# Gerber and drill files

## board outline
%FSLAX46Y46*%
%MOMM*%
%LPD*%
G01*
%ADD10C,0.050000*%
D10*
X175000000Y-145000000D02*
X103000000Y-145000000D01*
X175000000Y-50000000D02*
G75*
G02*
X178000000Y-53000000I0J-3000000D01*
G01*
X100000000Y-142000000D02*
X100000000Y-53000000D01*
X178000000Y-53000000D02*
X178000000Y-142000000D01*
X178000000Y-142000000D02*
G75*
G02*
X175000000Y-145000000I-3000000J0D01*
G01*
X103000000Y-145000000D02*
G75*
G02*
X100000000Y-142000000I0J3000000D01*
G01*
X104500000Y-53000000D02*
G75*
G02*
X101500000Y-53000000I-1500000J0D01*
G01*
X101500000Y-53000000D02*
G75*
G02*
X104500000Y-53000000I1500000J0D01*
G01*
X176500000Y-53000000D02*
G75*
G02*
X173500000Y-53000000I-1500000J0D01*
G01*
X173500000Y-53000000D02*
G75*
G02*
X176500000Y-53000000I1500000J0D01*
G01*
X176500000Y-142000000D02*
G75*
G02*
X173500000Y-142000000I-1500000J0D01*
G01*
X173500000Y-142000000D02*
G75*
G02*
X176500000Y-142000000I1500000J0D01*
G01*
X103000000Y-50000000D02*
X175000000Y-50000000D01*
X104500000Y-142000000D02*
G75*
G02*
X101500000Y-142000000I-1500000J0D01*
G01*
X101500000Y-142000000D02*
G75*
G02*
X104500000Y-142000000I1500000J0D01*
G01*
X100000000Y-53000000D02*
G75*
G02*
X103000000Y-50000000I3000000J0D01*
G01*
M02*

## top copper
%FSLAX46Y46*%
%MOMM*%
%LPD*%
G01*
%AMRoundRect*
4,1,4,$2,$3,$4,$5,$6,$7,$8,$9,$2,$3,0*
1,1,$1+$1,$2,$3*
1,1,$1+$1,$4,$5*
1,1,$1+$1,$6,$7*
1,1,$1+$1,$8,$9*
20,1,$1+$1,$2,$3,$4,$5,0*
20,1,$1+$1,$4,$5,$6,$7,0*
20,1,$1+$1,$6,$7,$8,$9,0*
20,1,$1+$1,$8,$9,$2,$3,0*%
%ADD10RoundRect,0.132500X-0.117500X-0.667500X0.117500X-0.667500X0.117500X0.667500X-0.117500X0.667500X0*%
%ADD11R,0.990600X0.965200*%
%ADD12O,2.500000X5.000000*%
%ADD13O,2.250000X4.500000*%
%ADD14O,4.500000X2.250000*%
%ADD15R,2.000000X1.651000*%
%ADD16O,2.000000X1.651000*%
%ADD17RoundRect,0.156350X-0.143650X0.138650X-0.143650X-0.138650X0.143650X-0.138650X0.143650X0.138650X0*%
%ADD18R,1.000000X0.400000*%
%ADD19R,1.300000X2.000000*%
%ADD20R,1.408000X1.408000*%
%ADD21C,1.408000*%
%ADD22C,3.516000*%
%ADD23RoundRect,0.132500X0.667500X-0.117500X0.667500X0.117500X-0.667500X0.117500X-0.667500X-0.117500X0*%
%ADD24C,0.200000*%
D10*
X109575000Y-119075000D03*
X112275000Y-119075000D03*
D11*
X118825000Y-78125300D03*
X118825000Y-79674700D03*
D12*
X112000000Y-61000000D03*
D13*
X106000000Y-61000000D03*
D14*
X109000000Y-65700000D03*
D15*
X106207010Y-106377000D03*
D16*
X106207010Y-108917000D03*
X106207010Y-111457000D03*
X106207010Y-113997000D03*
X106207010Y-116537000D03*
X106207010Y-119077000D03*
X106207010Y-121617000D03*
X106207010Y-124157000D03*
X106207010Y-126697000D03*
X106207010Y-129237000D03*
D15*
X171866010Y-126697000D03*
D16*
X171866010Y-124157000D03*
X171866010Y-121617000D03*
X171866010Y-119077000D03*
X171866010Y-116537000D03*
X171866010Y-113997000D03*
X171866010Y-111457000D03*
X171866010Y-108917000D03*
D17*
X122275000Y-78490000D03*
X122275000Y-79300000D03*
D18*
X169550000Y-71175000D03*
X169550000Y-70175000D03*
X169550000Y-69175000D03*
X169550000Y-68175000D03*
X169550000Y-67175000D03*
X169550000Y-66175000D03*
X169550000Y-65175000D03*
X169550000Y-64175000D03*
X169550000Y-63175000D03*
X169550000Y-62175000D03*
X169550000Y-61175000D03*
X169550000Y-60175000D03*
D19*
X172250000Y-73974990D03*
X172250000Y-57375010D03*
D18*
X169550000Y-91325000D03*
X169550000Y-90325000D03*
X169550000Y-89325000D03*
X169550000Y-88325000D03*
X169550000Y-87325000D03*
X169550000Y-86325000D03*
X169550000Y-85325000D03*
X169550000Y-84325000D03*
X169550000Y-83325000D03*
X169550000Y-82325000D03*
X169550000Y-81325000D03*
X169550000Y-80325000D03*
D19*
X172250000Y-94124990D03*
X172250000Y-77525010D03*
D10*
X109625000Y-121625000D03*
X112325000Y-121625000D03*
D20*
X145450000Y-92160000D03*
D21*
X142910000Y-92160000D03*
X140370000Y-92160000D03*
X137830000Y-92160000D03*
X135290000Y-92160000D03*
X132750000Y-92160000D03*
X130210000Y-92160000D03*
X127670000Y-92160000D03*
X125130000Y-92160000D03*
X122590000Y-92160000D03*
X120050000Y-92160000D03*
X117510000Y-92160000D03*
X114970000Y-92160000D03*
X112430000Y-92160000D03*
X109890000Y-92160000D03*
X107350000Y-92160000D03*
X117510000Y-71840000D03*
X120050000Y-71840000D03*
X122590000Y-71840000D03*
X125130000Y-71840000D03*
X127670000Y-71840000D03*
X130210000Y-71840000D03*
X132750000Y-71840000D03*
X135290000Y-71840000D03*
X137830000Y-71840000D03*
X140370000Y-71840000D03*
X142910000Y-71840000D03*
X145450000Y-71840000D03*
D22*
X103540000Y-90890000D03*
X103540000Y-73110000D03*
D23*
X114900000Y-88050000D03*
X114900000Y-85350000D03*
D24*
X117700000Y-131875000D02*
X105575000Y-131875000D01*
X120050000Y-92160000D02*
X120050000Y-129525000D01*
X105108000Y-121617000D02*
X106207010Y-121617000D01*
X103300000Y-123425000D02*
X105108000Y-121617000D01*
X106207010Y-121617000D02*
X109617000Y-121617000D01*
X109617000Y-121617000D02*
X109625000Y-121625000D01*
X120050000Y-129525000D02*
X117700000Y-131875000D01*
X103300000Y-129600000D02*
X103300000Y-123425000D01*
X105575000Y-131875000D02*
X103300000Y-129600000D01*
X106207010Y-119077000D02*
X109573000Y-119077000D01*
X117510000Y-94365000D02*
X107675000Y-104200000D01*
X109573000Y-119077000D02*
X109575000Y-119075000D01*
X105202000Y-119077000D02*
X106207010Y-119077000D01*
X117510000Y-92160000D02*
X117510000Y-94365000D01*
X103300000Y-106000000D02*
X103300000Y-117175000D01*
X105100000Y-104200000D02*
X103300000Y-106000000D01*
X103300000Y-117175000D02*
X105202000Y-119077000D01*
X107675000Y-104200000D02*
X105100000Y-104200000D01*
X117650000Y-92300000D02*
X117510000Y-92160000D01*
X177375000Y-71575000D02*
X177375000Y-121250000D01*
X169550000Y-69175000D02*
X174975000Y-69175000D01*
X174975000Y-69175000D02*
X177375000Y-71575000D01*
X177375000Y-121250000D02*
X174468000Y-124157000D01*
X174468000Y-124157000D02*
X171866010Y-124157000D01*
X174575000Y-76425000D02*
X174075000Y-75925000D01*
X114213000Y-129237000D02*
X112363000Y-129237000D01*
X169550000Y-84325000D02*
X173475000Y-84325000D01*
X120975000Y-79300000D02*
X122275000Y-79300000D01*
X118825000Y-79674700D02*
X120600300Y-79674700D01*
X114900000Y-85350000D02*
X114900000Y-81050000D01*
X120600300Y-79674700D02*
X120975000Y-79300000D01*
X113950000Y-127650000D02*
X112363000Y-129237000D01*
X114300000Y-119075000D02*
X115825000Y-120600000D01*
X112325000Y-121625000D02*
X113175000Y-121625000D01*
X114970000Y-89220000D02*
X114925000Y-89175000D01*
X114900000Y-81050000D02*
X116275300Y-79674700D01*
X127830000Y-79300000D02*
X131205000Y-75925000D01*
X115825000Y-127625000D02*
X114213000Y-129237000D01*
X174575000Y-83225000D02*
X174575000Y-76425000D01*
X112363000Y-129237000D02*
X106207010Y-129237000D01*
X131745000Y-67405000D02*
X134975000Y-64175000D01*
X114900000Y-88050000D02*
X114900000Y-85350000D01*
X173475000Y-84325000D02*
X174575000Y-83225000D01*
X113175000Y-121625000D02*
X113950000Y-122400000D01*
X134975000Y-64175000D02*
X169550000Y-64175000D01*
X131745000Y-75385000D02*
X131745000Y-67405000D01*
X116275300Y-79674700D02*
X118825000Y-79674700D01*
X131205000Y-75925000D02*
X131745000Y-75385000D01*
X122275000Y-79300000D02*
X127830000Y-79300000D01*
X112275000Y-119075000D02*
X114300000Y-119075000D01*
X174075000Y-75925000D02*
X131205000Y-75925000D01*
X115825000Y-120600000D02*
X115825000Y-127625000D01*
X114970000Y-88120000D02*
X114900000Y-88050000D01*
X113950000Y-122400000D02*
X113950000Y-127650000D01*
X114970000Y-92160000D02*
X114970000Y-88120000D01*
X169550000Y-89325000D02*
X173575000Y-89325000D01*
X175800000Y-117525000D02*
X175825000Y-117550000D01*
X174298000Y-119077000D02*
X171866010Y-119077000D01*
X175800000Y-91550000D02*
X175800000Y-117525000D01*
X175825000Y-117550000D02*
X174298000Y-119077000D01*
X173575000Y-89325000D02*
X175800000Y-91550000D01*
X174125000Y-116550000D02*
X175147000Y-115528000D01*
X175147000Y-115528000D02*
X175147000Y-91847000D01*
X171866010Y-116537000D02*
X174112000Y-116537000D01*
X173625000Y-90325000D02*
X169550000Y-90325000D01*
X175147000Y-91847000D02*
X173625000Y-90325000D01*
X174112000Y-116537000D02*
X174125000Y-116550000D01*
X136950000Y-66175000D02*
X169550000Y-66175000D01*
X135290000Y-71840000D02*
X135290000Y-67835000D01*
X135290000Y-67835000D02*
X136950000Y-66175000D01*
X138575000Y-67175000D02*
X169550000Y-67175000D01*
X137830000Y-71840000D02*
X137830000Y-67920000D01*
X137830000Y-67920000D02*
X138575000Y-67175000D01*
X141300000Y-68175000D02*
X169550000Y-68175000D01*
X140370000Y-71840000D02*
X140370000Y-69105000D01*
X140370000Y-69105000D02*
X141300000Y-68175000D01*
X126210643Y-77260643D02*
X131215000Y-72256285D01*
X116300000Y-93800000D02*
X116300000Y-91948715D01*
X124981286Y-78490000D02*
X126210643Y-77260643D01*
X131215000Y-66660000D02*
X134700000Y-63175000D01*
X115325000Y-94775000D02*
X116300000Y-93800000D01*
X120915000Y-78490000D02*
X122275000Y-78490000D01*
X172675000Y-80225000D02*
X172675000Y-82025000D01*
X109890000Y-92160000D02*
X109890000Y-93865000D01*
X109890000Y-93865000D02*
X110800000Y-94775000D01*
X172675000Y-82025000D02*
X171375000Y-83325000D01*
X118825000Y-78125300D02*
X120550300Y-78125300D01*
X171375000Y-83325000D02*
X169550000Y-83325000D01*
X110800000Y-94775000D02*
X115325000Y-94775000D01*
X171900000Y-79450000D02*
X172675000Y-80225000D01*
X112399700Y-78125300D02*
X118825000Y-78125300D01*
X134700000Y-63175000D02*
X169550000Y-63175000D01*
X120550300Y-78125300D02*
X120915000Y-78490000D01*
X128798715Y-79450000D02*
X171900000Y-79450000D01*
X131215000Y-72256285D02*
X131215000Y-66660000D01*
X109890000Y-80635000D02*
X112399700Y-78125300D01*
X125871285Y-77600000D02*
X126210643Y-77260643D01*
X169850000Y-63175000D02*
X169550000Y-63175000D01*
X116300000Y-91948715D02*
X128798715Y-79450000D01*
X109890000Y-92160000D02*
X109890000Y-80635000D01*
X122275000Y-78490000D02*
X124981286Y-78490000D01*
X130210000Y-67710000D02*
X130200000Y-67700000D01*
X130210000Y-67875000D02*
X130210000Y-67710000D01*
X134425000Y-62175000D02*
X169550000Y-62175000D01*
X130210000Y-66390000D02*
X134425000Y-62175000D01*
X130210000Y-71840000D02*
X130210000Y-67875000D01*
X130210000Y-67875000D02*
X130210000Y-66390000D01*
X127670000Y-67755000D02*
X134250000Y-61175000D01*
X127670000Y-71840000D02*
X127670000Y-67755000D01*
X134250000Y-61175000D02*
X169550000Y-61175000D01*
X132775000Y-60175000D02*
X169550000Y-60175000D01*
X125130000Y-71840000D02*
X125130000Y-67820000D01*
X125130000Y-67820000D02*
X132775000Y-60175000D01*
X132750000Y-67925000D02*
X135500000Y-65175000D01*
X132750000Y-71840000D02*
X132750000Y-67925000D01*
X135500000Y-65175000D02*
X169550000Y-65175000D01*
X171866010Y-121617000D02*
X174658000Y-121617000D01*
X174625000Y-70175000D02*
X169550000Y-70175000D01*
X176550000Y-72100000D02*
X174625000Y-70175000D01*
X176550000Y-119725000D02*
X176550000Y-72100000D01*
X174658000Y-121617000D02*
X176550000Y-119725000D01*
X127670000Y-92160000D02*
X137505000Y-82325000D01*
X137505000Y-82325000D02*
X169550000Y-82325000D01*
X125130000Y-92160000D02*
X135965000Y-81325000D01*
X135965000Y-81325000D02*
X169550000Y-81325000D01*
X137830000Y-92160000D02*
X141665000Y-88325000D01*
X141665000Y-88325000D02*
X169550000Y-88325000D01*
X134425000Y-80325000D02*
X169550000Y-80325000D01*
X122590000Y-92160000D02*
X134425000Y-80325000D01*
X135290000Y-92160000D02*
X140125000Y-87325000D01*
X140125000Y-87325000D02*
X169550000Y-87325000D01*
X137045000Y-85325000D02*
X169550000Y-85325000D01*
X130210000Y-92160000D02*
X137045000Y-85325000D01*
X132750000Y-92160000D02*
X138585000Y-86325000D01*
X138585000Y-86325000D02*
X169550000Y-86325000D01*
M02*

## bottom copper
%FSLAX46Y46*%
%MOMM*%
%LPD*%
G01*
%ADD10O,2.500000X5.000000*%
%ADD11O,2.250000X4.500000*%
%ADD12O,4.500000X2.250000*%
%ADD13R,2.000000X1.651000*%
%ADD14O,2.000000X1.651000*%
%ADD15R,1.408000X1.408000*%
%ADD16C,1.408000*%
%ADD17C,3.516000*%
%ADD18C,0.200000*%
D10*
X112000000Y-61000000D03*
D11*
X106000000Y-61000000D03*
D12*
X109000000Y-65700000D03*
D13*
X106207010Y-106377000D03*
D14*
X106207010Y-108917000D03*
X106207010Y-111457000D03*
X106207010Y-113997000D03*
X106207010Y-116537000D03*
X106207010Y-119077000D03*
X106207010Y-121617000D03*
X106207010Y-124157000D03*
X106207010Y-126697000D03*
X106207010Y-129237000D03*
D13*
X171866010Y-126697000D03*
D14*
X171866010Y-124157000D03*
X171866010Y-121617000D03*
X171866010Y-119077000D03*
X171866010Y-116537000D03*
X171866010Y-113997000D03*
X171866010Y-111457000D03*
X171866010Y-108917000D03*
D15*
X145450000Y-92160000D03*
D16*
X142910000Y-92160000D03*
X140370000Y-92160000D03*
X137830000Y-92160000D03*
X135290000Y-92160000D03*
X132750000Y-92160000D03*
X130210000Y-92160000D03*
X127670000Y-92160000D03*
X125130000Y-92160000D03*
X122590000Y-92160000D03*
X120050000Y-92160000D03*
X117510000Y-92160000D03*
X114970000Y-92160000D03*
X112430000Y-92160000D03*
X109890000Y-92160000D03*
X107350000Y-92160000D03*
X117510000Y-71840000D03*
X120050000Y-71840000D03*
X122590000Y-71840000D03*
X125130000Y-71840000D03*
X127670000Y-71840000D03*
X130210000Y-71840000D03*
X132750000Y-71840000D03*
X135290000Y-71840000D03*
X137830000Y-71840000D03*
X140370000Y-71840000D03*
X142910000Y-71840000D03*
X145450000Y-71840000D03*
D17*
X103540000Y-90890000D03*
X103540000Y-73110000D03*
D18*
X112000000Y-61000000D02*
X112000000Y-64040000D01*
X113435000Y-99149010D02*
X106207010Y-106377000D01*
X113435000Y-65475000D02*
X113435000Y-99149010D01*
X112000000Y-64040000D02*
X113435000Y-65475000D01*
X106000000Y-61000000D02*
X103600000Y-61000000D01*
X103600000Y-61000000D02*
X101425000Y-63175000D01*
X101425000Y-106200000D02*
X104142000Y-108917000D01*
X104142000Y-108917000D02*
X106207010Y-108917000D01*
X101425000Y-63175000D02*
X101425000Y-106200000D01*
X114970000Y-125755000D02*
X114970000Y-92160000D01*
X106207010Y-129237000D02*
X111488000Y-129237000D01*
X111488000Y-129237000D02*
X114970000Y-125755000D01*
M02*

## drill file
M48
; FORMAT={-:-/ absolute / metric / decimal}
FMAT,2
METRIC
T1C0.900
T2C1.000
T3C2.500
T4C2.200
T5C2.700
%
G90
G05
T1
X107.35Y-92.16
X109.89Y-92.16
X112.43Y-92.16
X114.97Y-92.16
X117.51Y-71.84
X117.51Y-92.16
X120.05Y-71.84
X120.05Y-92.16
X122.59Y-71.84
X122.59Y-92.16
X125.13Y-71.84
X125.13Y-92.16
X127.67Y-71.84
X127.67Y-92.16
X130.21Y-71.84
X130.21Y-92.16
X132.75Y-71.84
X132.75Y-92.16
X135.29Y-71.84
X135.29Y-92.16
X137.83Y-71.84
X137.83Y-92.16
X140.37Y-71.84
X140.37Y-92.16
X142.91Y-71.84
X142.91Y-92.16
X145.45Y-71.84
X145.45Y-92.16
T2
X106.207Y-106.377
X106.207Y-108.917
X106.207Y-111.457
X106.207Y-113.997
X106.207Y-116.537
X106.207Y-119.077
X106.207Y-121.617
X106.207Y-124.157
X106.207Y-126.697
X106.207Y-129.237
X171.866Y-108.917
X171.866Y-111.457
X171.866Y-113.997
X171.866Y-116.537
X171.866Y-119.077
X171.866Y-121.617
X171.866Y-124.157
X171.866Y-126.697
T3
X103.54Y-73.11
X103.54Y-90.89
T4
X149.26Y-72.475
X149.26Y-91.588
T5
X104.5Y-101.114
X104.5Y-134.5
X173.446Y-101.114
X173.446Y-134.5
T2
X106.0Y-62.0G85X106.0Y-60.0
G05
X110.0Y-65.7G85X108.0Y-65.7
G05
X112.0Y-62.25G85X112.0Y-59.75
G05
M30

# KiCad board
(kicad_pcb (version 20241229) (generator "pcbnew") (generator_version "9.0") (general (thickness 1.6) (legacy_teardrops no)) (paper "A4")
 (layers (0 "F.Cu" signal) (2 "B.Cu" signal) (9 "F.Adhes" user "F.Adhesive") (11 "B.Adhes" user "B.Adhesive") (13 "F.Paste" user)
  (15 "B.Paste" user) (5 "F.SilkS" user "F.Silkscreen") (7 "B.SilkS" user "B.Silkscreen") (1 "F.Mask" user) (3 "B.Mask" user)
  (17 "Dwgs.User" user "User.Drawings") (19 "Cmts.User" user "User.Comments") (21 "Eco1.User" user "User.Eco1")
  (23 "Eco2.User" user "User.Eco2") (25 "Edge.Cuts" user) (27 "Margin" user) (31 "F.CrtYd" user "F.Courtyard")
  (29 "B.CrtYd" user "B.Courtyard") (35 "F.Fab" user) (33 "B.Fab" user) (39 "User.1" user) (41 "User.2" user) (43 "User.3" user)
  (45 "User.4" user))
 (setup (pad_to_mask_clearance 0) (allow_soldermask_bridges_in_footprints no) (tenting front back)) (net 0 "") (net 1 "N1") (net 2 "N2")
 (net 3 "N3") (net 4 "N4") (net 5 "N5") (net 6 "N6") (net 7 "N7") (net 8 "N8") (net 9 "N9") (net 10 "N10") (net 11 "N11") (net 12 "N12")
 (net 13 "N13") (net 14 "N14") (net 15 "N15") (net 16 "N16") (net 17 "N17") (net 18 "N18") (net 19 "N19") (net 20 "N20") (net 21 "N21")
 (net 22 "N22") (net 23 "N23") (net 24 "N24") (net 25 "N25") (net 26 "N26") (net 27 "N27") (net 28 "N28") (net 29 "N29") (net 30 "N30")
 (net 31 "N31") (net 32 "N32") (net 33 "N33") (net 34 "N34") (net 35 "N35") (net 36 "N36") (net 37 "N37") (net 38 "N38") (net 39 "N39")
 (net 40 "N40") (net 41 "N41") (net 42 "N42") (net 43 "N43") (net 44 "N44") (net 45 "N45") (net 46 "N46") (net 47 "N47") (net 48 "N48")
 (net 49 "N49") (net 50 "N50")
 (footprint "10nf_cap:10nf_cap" (layer "F.Cu") (at 109.575 119.075)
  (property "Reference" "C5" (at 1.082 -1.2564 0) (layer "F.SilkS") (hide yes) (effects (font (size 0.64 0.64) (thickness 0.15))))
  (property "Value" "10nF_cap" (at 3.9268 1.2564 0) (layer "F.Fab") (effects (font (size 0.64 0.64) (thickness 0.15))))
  (pad "1" smd roundrect (at 0 0) (size 0.5 1.6) (layers "F.Cu" "F.Mask" "F.Paste") (roundrect_rratio 0.265) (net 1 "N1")
   (solder_mask_margin 0.102))
  (pad "2" smd roundrect (at 2.7 0) (size 0.5 1.6) (layers "F.Cu" "F.Mask" "F.Paste") (roundrect_rratio 0.265) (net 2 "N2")
   (solder_mask_margin 0.102)))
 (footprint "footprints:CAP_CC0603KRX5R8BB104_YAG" (layer "F.Cu") (at 118.825 78.9 -90)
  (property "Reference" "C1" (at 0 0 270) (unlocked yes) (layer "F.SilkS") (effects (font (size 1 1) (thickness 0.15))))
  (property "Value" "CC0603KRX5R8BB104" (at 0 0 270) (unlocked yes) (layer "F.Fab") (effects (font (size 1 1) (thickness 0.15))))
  (pad "1" smd rect (at -0.7747 0 270) (size 0.9652 0.9906) (layers "F.Cu" "F.Mask" "F.Paste") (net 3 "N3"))
  (pad "2" smd rect (at 0.7747 0 270) (size 0.9652 0.9906) (layers "F.Cu" "F.Mask" "F.Paste") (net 2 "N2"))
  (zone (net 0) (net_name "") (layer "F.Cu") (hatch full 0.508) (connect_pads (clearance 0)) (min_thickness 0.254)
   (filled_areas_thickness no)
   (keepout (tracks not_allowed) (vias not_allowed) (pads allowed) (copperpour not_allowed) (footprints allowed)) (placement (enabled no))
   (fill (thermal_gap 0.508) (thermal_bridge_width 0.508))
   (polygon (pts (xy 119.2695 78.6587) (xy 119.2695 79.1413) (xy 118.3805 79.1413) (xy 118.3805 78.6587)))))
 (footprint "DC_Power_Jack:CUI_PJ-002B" (layer "F.Cu") (at 112 61 180)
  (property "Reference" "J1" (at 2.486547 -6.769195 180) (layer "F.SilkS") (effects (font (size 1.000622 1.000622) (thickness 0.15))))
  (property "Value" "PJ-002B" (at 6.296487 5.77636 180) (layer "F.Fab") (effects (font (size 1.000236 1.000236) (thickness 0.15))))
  (pad "1" thru_hole oval (at 0 0 180) (size 2.5 5) (drill oval 1 3.5) (layers "*.Cu" "*.Mask") (remove_unused_layers no) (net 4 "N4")
   (solder_mask_margin 0.102))
  (pad "2" thru_hole oval (at 6 0 180) (size 2.25 4.5) (drill oval 1 3) (layers "*.Cu" "*.Mask") (remove_unused_layers no) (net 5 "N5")
   (solder_mask_margin 0.102))
  (pad "3" thru_hole oval (at 3 -4.7 180) (size 4.5 2.25) (drill oval 3 1) (layers "*.Cu" "*.Mask") (remove_unused_layers no) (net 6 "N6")
   (solder_mask_margin 0.102)))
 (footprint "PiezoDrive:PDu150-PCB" (layer "F.Cu") (at 101 138)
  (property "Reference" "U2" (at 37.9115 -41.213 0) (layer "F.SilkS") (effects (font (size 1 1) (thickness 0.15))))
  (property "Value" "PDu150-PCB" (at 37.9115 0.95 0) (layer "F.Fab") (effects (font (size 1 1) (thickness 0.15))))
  (pad "" np_thru_hole circle (at 3.5 -36.886 270) (size 1.524 1.524) (drill 2.7) (layers "*.Cu" "*.Mask") (thermal_bridge_angle 90))
  (pad "" np_thru_hole circle (at 3.5 -3.5) (size 1.524 1.524) (drill 2.7) (layers "*.Cu" "*.Mask") (thermal_bridge_angle 90))
  (pad "" np_thru_hole circle (at 72.446 -36.886 180) (size 1.524 1.524) (drill 2.7) (layers "*.Cu" "*.Mask") (thermal_bridge_angle 90))
  (pad "" np_thru_hole circle (at 72.446 -3.5 90) (size 1.524 1.524) (drill 2.7) (layers "*.Cu" "*.Mask") (thermal_bridge_angle 90))
  (pad "1" thru_hole rect (at 5.20701 -31.623 270) (size 1.651 2) (drill 1) (layers "*.Cu" "*.Mask") (remove_unused_layers no) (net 4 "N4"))
  (pad "2" thru_hole oval (at 5.20701 -29.083 270) (size 1.651 2) (drill 1) (layers "*.Cu" "*.Mask") (remove_unused_layers no) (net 5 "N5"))
  (pad "3" thru_hole oval (at 5.20701 -26.543 270) (size 1.651 2) (drill 1) (layers "*.Cu" "*.Mask") (remove_unused_layers no) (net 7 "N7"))
  (pad "4" thru_hole oval (at 5.20701 -24.003 270) (size 1.651 2) (drill 1) (layers "*.Cu" "*.Mask") (remove_unused_layers no) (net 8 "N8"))
  (pad "5" thru_hole oval (at 5.20701 -21.463 270) (size 1.651 2) (drill 1) (layers "*.Cu" "*.Mask") (remove_unused_layers no) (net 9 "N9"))
  (pad "6" thru_hole oval (at 5.20701 -18.923 270) (size 1.651 2) (drill 1) (layers "*.Cu" "*.Mask") (remove_unused_layers no) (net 1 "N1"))
  (pad "7" thru_hole oval (at 5.20701 -16.383 270) (size 1.651 2) (drill 1) (layers "*.Cu" "*.Mask") (remove_unused_layers no)
   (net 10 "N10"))
  (pad "8" thru_hole oval (at 5.20701 -13.843 270) (size 1.651 2) (drill 1) (layers "*.Cu" "*.Mask") (remove_unused_layers no)
   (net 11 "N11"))
  (pad "9" thru_hole oval (at 5.20701 -11.303 270) (size 1.651 2) (drill 1) (layers "*.Cu" "*.Mask") (remove_unused_layers no)
   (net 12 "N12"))
  (pad "10" thru_hole oval (at 5.20701 -8.763 270) (size 1.651 2) (drill 1) (layers "*.Cu" "*.Mask") (remove_unused_layers no) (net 2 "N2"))
  (pad "11" thru_hole rect (at 70.86601 -11.303 90) (size 1.651 2) (drill 1) (layers "*.Cu" "*.Mask") (remove_unused_layers no)
   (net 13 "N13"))
  (pad "12" thru_hole oval (at 70.86601 -13.843 90) (size 1.651 2) (drill 1) (layers "*.Cu" "*.Mask") (remove_unused_layers no)
   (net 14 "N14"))
  (pad "13" thru_hole oval (at 70.86601 -16.383 90) (size 1.651 2) (drill 1) (layers "*.Cu" "*.Mask") (remove_unused_layers no)
   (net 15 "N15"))
  (pad "14" thru_hole oval (at 70.86601 -18.923 90) (size 1.651 2) (drill 1) (layers "*.Cu" "*.Mask") (remove_unused_layers no)
   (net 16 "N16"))
  (pad "15" thru_hole oval (at 70.86601 -21.463 90) (size 1.651 2) (drill 1) (layers "*.Cu" "*.Mask") (remove_unused_layers no)
   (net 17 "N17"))
  (pad "16" thru_hole oval (at 70.86601 -24.003 90) (size 1.651 2) (drill 1) (layers "*.Cu" "*.Mask") (remove_unused_layers no)
   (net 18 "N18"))
  (pad "17" thru_hole oval (at 70.86601 -26.543 90) (size 1.651 2) (drill 1) (layers "*.Cu" "*.Mask") (remove_unused_layers no)
   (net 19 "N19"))
  (pad "18" thru_hole oval (at 70.86601 -29.083 90) (size 1.651 2) (drill 1) (layers "*.Cu" "*.Mask") (remove_unused_layers no)
   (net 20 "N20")))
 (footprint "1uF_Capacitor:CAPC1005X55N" (layer "F.Cu") (at 122.275 78.895 -90)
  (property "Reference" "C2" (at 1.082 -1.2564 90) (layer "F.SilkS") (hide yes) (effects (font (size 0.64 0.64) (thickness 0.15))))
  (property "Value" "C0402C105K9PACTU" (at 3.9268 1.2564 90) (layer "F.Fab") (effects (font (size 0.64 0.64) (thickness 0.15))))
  (pad "1" smd roundrect (at -0.405 0 270) (size 0.59 0.6) (layers "F.Cu" "F.Mask" "F.Paste") (roundrect_rratio 0.265) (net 3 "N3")
   (solder_mask_margin 0.102))
  (pad "2" smd roundrect (at 0.405 0 270) (size 0.59 0.6) (layers "F.Cu" "F.Mask" "F.Paste") (roundrect_rratio 0.265) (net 2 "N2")
   (solder_mask_margin 0.102)))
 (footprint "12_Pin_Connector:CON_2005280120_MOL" (layer "F.Cu") (at 172 65.675 90)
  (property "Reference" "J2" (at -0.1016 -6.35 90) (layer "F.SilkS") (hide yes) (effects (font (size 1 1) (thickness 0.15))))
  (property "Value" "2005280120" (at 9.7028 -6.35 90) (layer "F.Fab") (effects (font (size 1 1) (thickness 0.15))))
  (pad "1" smd rect (at -5.5 -2.45 90) (size 0.4 1) (layers "F.Cu" "F.Mask" "F.Paste") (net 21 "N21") (solder_mask_margin 0.102))
  (pad "2" smd rect (at -4.5 -2.45 90) (size 0.4 1) (layers "F.Cu" "F.Mask" "F.Paste") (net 15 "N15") (solder_mask_margin 0.102))
  (pad "3" smd rect (at -3.5 -2.45 90) (size 0.4 1) (layers "F.Cu" "F.Mask" "F.Paste") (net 14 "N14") (solder_mask_margin 0.102))
  (pad "4" smd rect (at -2.5 -2.45 90) (size 0.4 1) (layers "F.Cu" "F.Mask" "F.Paste") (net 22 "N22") (solder_mask_margin 0.102))
  (pad "5" smd rect (at -1.5 -2.45 90) (size 0.4 1) (layers "F.Cu" "F.Mask" "F.Paste") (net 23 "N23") (solder_mask_margin 0.102))
  (pad "6" smd rect (at -0.5 -2.45 90) (size 0.4 1) (layers "F.Cu" "F.Mask" "F.Paste") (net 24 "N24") (solder_mask_margin 0.102))
  (pad "7" smd rect (at 0.5 -2.45 90) (size 0.4 1) (layers "F.Cu" "F.Mask" "F.Paste") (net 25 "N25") (solder_mask_margin 0.102))
  (pad "8" smd rect (at 1.5 -2.45 90) (size 0.4 1) (layers "F.Cu" "F.Mask" "F.Paste") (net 2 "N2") (solder_mask_margin 0.102))
  (pad "9" smd rect (at 2.5 -2.45 90) (size 0.4 1) (layers "F.Cu" "F.Mask" "F.Paste") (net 3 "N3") (solder_mask_margin 0.102))
  (pad "10" smd rect (at 3.5 -2.45 90) (size 0.4 1) (layers "F.Cu" "F.Mask" "F.Paste") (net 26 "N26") (solder_mask_margin 0.102))
  (pad "11" smd rect (at 4.5 -2.45 90) (size 0.4 1) (layers "F.Cu" "F.Mask" "F.Paste") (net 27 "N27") (solder_mask_margin 0.102))
  (pad "12" smd rect (at 5.5 -2.45 90) (size 0.4 1) (layers "F.Cu" "F.Mask" "F.Paste") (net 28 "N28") (solder_mask_margin 0.102))
  (pad "P1" smd rect (at -8.29999 0.25 90) (size 2 1.3) (layers "F.Cu" "F.Mask" "F.Paste") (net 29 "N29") (solder_mask_margin 0.102))
  (pad "P2" smd rect (at 8.29999 0.25 90) (size 2 1.3) (layers "F.Cu" "F.Mask" "F.Paste") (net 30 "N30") (solder_mask_margin 0.102)))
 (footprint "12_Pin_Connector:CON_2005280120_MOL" (layer "F.Cu") (at 172 85.825 90)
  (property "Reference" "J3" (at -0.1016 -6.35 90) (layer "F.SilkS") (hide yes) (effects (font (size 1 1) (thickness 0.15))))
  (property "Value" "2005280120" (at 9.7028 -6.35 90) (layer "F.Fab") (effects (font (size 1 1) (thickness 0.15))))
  (pad "1" smd rect (at -5.5 -2.45 90) (size 0.4 1) (layers "F.Cu" "F.Mask" "F.Paste") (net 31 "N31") (solder_mask_margin 0.102))
  (pad "2" smd rect (at -4.5 -2.45 90) (size 0.4 1) (layers "F.Cu" "F.Mask" "F.Paste") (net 17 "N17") (solder_mask_margin 0.102))
  (pad "3" smd rect (at -3.5 -2.45 90) (size 0.4 1) (layers "F.Cu" "F.Mask" "F.Paste") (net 16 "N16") (solder_mask_margin 0.102))
  (pad "4" smd rect (at -2.5 -2.45 90) (size 0.4 1) (layers "F.Cu" "F.Mask" "F.Paste") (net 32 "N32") (solder_mask_margin 0.102))
  (pad "5" smd rect (at -1.5 -2.45 90) (size 0.4 1) (layers "F.Cu" "F.Mask" "F.Paste") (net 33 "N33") (solder_mask_margin 0.102))
  (pad "6" smd rect (at -0.5 -2.45 90) (size 0.4 1) (layers "F.Cu" "F.Mask" "F.Paste") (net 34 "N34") (solder_mask_margin 0.102))
  (pad "7" smd rect (at 0.5 -2.45 90) (size 0.4 1) (layers "F.Cu" "F.Mask" "F.Paste") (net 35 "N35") (solder_mask_margin 0.102))
  (pad "8" smd rect (at 1.5 -2.45 90) (size 0.4 1) (layers "F.Cu" "F.Mask" "F.Paste") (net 2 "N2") (solder_mask_margin 0.102))
  (pad "9" smd rect (at 2.5 -2.45 90) (size 0.4 1) (layers "F.Cu" "F.Mask" "F.Paste") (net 3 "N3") (solder_mask_margin 0.102))
  (pad "10" smd rect (at 3.5 -2.45 90) (size 0.4 1) (layers "F.Cu" "F.Mask" "F.Paste") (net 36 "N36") (solder_mask_margin 0.102))
  (pad "11" smd rect (at 4.5 -2.45 90) (size 0.4 1) (layers "F.Cu" "F.Mask" "F.Paste") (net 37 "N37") (solder_mask_margin 0.102))
  (pad "12" smd rect (at 5.5 -2.45 90) (size 0.4 1) (layers "F.Cu" "F.Mask" "F.Paste") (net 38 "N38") (solder_mask_margin 0.102))
  (pad "P1" smd rect (at -8.29999 0.25 90) (size 2 1.3) (layers "F.Cu" "F.Mask" "F.Paste") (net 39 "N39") (solder_mask_margin 0.102))
  (pad "P2" smd rect (at 8.29999 0.25 90) (size 2 1.3) (layers "F.Cu" "F.Mask" "F.Paste") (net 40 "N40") (solder_mask_margin 0.102)))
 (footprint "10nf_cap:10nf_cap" (layer "F.Cu") (at 109.625 121.625)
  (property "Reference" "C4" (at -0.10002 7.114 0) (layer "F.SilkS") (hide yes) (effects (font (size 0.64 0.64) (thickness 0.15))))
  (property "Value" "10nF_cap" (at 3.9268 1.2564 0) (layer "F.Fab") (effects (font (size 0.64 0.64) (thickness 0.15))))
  (pad "1" smd roundrect (at 0 0) (size 0.5 1.6) (layers "F.Cu" "F.Mask" "F.Paste") (roundrect_rratio 0.265) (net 10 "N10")
   (solder_mask_margin 0.102))
  (pad "2" smd roundrect (at 2.7 0) (size 0.5 1.6) (layers "F.Cu" "F.Mask" "F.Paste") (roundrect_rratio 0.265) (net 2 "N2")
   (solder_mask_margin 0.102)))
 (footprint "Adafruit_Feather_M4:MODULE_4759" (layer "F.Cu") (at 126.4 82)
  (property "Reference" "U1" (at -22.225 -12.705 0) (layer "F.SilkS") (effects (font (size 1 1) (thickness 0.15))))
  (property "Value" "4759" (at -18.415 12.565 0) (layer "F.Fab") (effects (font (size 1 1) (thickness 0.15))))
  (pad "" np_thru_hole circle (at 22.86 -9.525) (size 2.2 2.2) (drill 2.2) (layers "*.Cu" "*.Mask"))
  (pad "" np_thru_hole circle (at 22.86 9.5885) (size 2.2 2.2) (drill 2.2) (layers "*.Cu" "*.Mask"))
  (pad "1" thru_hole rect (at 19.05 10.16) (size 1.408 1.408) (drill 0.9) (layers "*.Cu" "*.Mask") (remove_unused_layers no) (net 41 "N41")
   (solder_mask_margin 0.102))
  (pad "2" thru_hole circle (at 16.51 10.16) (size 1.408 1.408) (drill 0.9) (layers "*.Cu" "*.Mask") (remove_unused_layers no)
   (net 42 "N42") (solder_mask_margin 0.102))
  (pad "3" thru_hole circle (at 13.97 10.16) (size 1.408 1.408) (drill 0.9) (layers "*.Cu" "*.Mask") (remove_unused_layers no)
   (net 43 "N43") (solder_mask_margin 0.102))
  (pad "4" thru_hole circle (at 11.43 10.16) (size 1.408 1.408) (drill 0.9) (layers "*.Cu" "*.Mask") (remove_unused_layers no)
   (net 32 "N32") (solder_mask_margin 0.102))
  (pad "5" thru_hole circle (at 8.89 10.16) (size 1.408 1.408) (drill 0.9) (layers "*.Cu" "*.Mask") (remove_unused_layers no) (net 33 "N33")
   (solder_mask_margin 0.102))
  (pad "6" thru_hole circle (at 6.35 10.16) (size 1.408 1.408) (drill 0.9) (layers "*.Cu" "*.Mask") (remove_unused_layers no) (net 34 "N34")
   (solder_mask_margin 0.102))
  (pad "7" thru_hole circle (at 3.81 10.16) (size 1.408 1.408) (drill 0.9) (layers "*.Cu" "*.Mask") (remove_unused_layers no) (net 35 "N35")
   (solder_mask_margin 0.102))
  (pad "8" thru_hole circle (at 1.27 10.16) (size 1.408 1.408) (drill 0.9) (layers "*.Cu" "*.Mask") (remove_unused_layers no) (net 36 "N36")
   (solder_mask_margin 0.102))
  (pad "9" thru_hole circle (at -1.27 10.16) (size 1.408 1.408) (drill 0.9) (layers "*.Cu" "*.Mask") (remove_unused_layers no)
   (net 37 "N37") (solder_mask_margin 0.102))
  (pad "10" thru_hole circle (at -3.81 10.16) (size 1.408 1.408) (drill 0.9) (layers "*.Cu" "*.Mask") (remove_unused_layers no)
   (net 38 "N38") (solder_mask_margin 0.102))
  (pad "11" thru_hole circle (at -6.35 10.16) (size 1.408 1.408) (drill 0.9) (layers "*.Cu" "*.Mask") (remove_unused_layers no)
   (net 10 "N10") (solder_mask_margin 0.102))
  (pad "12" thru_hole circle (at -8.89 10.16) (size 1.408 1.408) (drill 0.9) (layers "*.Cu" "*.Mask") (remove_unused_layers no) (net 1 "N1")
   (solder_mask_margin 0.102))
  (pad "13" thru_hole circle (at -11.43 10.16) (size 1.408 1.408) (drill 0.9) (layers "*.Cu" "*.Mask") (remove_unused_layers no)
   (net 2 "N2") (solder_mask_margin 0.102))
  (pad "14" thru_hole circle (at -13.97 10.16) (size 1.408 1.408) (drill 0.9) (layers "*.Cu" "*.Mask") (remove_unused_layers no)
   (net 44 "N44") (solder_mask_margin 0.102))
  (pad "15" thru_hole circle (at -16.51 10.16) (size 1.408 1.408) (drill 0.9) (layers "*.Cu" "*.Mask") (remove_unused_layers no)
   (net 3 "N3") (solder_mask_margin 0.102))
  (pad "16" thru_hole circle (at -19.05 10.16) (size 1.408 1.408) (drill 0.9) (layers "*.Cu" "*.Mask") (remove_unused_layers no)
   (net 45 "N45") (solder_mask_margin 0.102))
  (pad "17" thru_hole circle (at -8.89 -10.16) (size 1.408 1.408) (drill 0.9) (layers "*.Cu" "*.Mask") (remove_unused_layers no)
   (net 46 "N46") (solder_mask_margin 0.102))
  (pad "18" thru_hole circle (at -6.35 -10.16) (size 1.408 1.408) (drill 0.9) (layers "*.Cu" "*.Mask") (remove_unused_layers no)
   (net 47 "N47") (solder_mask_margin 0.102))
  (pad "19" thru_hole circle (at -3.81 -10.16) (size 1.408 1.408) (drill 0.9) (layers "*.Cu" "*.Mask") (remove_unused_layers no)
   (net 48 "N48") (solder_mask_margin 0.102))
  (pad "20" thru_hole circle (at -1.27 -10.16) (size 1.408 1.408) (drill 0.9) (layers "*.Cu" "*.Mask") (remove_unused_layers no)
   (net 28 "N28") (solder_mask_margin 0.102))
  (pad "21" thru_hole circle (at 1.27 -10.16) (size 1.408 1.408) (drill 0.9) (layers "*.Cu" "*.Mask") (remove_unused_layers no)
   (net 27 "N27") (solder_mask_margin 0.102))
  (pad "22" thru_hole circle (at 3.81 -10.16) (size 1.408 1.408) (drill 0.9) (layers "*.Cu" "*.Mask") (remove_unused_layers no)
   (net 26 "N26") (solder_mask_margin 0.102))
  (pad "23" thru_hole circle (at 6.35 -10.16) (size 1.408 1.408) (drill 0.9) (layers "*.Cu" "*.Mask") (remove_unused_layers no)
   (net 25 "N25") (solder_mask_margin 0.102))
  (pad "24" thru_hole circle (at 8.89 -10.16) (size 1.408 1.408) (drill 0.9) (layers "*.Cu" "*.Mask") (remove_unused_layers no)
   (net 24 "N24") (solder_mask_margin 0.102))
  (pad "25" thru_hole circle (at 11.43 -10.16) (size 1.408 1.408) (drill 0.9) (layers "*.Cu" "*.Mask") (remove_unused_layers no)
   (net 23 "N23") (solder_mask_margin 0.102))
  (pad "26" thru_hole circle (at 13.97 -10.16) (size 1.408 1.408) (drill 0.9) (layers "*.Cu" "*.Mask") (remove_unused_layers no)
   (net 22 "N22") (solder_mask_margin 0.102))
  (pad "27" thru_hole circle (at 16.51 -10.16) (size 1.408 1.408) (drill 0.9) (layers "*.Cu" "*.Mask") (remove_unused_layers no)
   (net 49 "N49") (solder_mask_margin 0.102))
  (pad "28" thru_hole circle (at 19.05 -10.16) (size 1.408 1.408) (drill 0.9) (layers "*.Cu" "*.Mask") (remove_unused_layers no)
   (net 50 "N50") (solder_mask_margin 0.102))
  (pad "P1" thru_hole circle (at -22.86 8.89) (size 3.516 3.516) (drill 2.5) (layers "*.Cu" "*.Mask") (remove_unused_layers no)
   (solder_mask_margin 0.102))
  (pad "P2" thru_hole circle (at -22.86 -8.89) (size 3.516 3.516) (drill 2.5) (layers "*.Cu" "*.Mask") (remove_unused_layers no)
   (solder_mask_margin 0.102)))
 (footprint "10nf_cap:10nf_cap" (layer "F.Cu") (at 114.9 88.05 90)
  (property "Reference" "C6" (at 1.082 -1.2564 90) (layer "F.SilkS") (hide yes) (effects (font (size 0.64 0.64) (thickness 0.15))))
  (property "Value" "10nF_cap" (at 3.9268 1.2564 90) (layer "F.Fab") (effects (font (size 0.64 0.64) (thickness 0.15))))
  (pad "1" smd roundrect (at 0 0 90) (size 0.5 1.6) (layers "F.Cu" "F.Mask" "F.Paste") (roundrect_rratio 0.265) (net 2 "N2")
   (solder_mask_margin 0.102))
  (pad "2" smd roundrect (at 2.7 0 90) (size 0.5 1.6) (layers "F.Cu" "F.Mask" "F.Paste") (roundrect_rratio 0.265) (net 2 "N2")
   (solder_mask_margin 0.102)))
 (gr_line (start 175 145) (end 103 145) (stroke (width 0.05) (type solid)) (layer "Edge.Cuts"))
 (gr_arc (start 175 50) (mid 177.12132 50.87868) (end 178 53) (stroke (width 0.05) (type default)) (layer "Edge.Cuts"))
 (gr_line (start 100 142) (end 100 53) (stroke (width 0.05) (type solid)) (layer "Edge.Cuts"))
 (gr_line (start 178 53) (end 178 142) (stroke (width 0.05) (type solid)) (layer "Edge.Cuts"))
 (gr_arc (start 178 142) (mid 177.12132 144.12132) (end 175 145) (stroke (width 0.05) (type default)) (layer "Edge.Cuts"))
 (gr_arc (start 103 145) (mid 100.87868 144.12132) (end 100 142) (stroke (width 0.05) (type default)) (layer "Edge.Cuts"))
 (gr_circle (center 103 53) (end 104.5 53) (stroke (width 0.05) (type solid)) (fill no) (layer "Edge.Cuts"))
 (gr_circle (center 175 53) (end 176.5 53) (stroke (width 0.05) (type solid)) (fill no) (layer "Edge.Cuts"))
 (gr_circle (center 175 142) (end 176.5 142) (stroke (width 0.05) (type solid)) (fill no) (layer "Edge.Cuts"))
 (gr_line (start 103 50) (end 175 50) (stroke (width 0.05) (type solid)) (layer "Edge.Cuts"))
 (gr_circle (center 103 142) (end 104.5 142) (stroke (width 0.05) (type solid)) (fill no) (layer "Edge.Cuts"))
 (gr_arc (start 100 53) (mid 100.87868 50.87868) (end 103 50) (stroke (width 0.05) (type default)) (layer "Edge.Cuts"))
 (segment (start 112 61) (end 112 64.04) (width 0.2) (layer "B.Cu") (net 4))
 (segment (start 113.435 99.14901) (end 106.20701 106.377) (width 0.2) (layer "B.Cu") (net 4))
 (segment (start 113.435 65.475) (end 113.435 99.14901) (width 0.2) (layer "B.Cu") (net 4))
 (segment (start 112 64.04) (end 113.435 65.475) (width 0.2) (layer "B.Cu") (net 4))
 (segment (start 106 61) (end 103.6 61) (width 0.2) (layer "B.Cu") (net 5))
 (segment (start 103.6 61) (end 101.425 63.175) (width 0.2) (layer "B.Cu") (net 5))
 (segment (start 101.425 106.2) (end 104.142 108.917) (width 0.2) (layer "B.Cu") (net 5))
 (segment (start 104.142 108.917) (end 106.20701 108.917) (width 0.2) (layer "B.Cu") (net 5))
 (segment (start 101.425 63.175) (end 101.425 106.2) (width 0.2) (layer "B.Cu") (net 5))
 (segment (start 117.7 131.875) (end 105.575 131.875) (width 0.2) (layer "F.Cu") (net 10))
 (segment (start 120.05 92.16) (end 120.05 129.525) (width 0.2) (layer "F.Cu") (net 10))
 (segment (start 105.108 121.617) (end 106.20701 121.617) (width 0.2) (layer "F.Cu") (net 10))
 (segment (start 103.3 123.425) (end 105.108 121.617) (width 0.2) (layer "F.Cu") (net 10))
 (segment (start 106.20701 121.617) (end 109.617 121.617) (width 0.2) (layer "F.Cu") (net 10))
 (segment (start 109.617 121.617) (end 109.625 121.625) (width 0.2) (layer "F.Cu") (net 10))
 (segment (start 120.05 129.525) (end 117.7 131.875) (width 0.2) (layer "F.Cu") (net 10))
 (segment (start 103.3 129.6) (end 103.3 123.425) (width 0.2) (layer "F.Cu") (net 10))
 (segment (start 105.575 131.875) (end 103.3 129.6) (width 0.2) (layer "F.Cu") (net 10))
 (segment (start 106.20701 119.077) (end 109.573 119.077) (width 0.2) (layer "F.Cu") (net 1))
 (segment (start 117.51 94.365) (end 107.675 104.2) (width 0.2) (layer "F.Cu") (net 1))
 (segment (start 109.573 119.077) (end 109.575 119.075) (width 0.2) (layer "F.Cu") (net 1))
 (segment (start 105.202 119.077) (end 106.20701 119.077) (width 0.2) (layer "F.Cu") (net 1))
 (segment (start 117.51 92.16) (end 117.51 94.365) (width 0.2) (layer "F.Cu") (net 1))
 (segment (start 103.3 106) (end 103.3 117.175) (width 0.2) (layer "F.Cu") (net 1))
 (segment (start 105.1 104.2) (end 103.3 106) (width 0.2) (layer "F.Cu") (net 1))
 (segment (start 103.3 117.175) (end 105.202 119.077) (width 0.2) (layer "F.Cu") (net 1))
 (segment (start 107.675 104.2) (end 105.1 104.2) (width 0.2) (layer "F.Cu") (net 1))
 (segment (start 117.65 92.3) (end 117.51 92.16) (width 0.2) (layer "F.Cu") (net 1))
 (segment (start 177.375 71.575) (end 177.375 121.25) (width 0.2) (layer "F.Cu") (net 14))
 (segment (start 169.55 69.175) (end 174.975 69.175) (width 0.2) (layer "F.Cu") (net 14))
 (segment (start 174.975 69.175) (end 177.375 71.575) (width 0.2) (layer "F.Cu") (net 14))
 (segment (start 177.375 121.25) (end 174.468 124.157) (width 0.2) (layer "F.Cu") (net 14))
 (segment (start 174.468 124.157) (end 171.86601 124.157) (width 0.2) (layer "F.Cu") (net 14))
 (segment (start 174.575 76.425) (end 174.075 75.925) (width 0.2) (layer "F.Cu") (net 2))
 (segment (start 114.213 129.237) (end 112.363 129.237) (width 0.2) (layer "F.Cu") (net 2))
 (segment (start 169.55 84.325) (end 173.475 84.325) (width 0.2) (layer "F.Cu") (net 2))
 (segment (start 120.975 79.3) (end 122.275 79.3) (width 0.2) (layer "F.Cu") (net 2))
 (segment (start 118.825 79.6747) (end 120.6003 79.6747) (width 0.2) (layer "F.Cu") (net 2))
 (segment (start 114.9 85.35) (end 114.9 81.05) (width 0.2) (layer "F.Cu") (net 2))
 (segment (start 120.6003 79.6747) (end 120.975 79.3) (width 0.2) (layer "F.Cu") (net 2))
 (segment (start 113.95 127.65) (end 112.363 129.237) (width 0.2) (layer "F.Cu") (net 2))
 (segment (start 114.3 119.075) (end 115.825 120.6) (width 0.2) (layer "F.Cu") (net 2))
 (segment (start 112.325 121.625) (end 113.175 121.625) (width 0.2) (layer "F.Cu") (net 2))
 (segment (start 114.97 89.22) (end 114.925 89.175) (width 0.2) (layer "F.Cu") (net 2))
 (segment (start 114.9 81.05) (end 116.2753 79.6747) (width 0.2) (layer "F.Cu") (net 2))
 (segment (start 127.83 79.3) (end 131.205 75.925) (width 0.2) (layer "F.Cu") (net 2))
 (segment (start 115.825 127.625) (end 114.213 129.237) (width 0.2) (layer "F.Cu") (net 2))
 (segment (start 174.575 83.225) (end 174.575 76.425) (width 0.2) (layer "F.Cu") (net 2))
 (segment (start 112.363 129.237) (end 106.20701 129.237) (width 0.2) (layer "F.Cu") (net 2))
 (segment (start 131.745 67.405) (end 134.975 64.175) (width 0.2) (layer "F.Cu") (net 2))
 (segment (start 114.9 88.05) (end 114.9 85.35) (width 0.2) (layer "F.Cu") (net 2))
 (segment (start 173.475 84.325) (end 174.575 83.225) (width 0.2) (layer "F.Cu") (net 2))
 (segment (start 113.175 121.625) (end 113.95 122.4) (width 0.2) (layer "F.Cu") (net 2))
 (segment (start 134.975 64.175) (end 169.55 64.175) (width 0.2) (layer "F.Cu") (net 2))
 (segment (start 131.745 75.385) (end 131.745 67.405) (width 0.2) (layer "F.Cu") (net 2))
 (segment (start 116.2753 79.6747) (end 118.825 79.6747) (width 0.2) (layer "F.Cu") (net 2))
 (segment (start 131.205 75.925) (end 131.745 75.385) (width 0.2) (layer "F.Cu") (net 2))
 (segment (start 122.275 79.3) (end 127.83 79.3) (width 0.2) (layer "F.Cu") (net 2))
 (segment (start 112.275 119.075) (end 114.3 119.075) (width 0.2) (layer "F.Cu") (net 2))
 (segment (start 174.075 75.925) (end 131.205 75.925) (width 0.2) (layer "F.Cu") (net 2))
 (segment (start 115.825 120.6) (end 115.825 127.625) (width 0.2) (layer "F.Cu") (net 2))
 (segment (start 114.97 88.12) (end 114.9 88.05) (width 0.2) (layer "F.Cu") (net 2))
 (segment (start 113.95 122.4) (end 113.95 127.65) (width 0.2) (layer "F.Cu") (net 2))
 (segment (start 114.97 92.16) (end 114.97 88.12) (width 0.2) (layer "F.Cu") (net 2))
 (segment (start 114.97 125.755) (end 114.97 92.16) (width 0.2) (layer "B.Cu") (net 2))
 (segment (start 106.20701 129.237) (end 111.488 129.237) (width 0.2) (layer "B.Cu") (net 2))
 (segment (start 111.488 129.237) (end 114.97 125.755) (width 0.2) (layer "B.Cu") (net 2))
 (segment (start 169.55 89.325) (end 173.575 89.325) (width 0.2) (layer "F.Cu") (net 16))
 (segment (start 175.8 117.525) (end 175.825 117.55) (width 0.2) (layer "F.Cu") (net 16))
 (segment (start 174.298 119.077) (end 171.86601 119.077) (width 0.2) (layer "F.Cu") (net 16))
 (segment (start 175.8 91.55) (end 175.8 117.525) (width 0.2) (layer "F.Cu") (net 16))
 (segment (start 175.825 117.55) (end 174.298 119.077) (width 0.2) (layer "F.Cu") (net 16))
 (segment (start 173.575 89.325) (end 175.8 91.55) (width 0.2) (layer "F.Cu") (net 16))
 (segment (start 174.125 116.55) (end 175.147 115.528) (width 0.2) (layer "F.Cu") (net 17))
 (segment (start 175.147 115.528) (end 175.147 91.847) (width 0.2) (layer "F.Cu") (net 17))
 (segment (start 171.86601 116.537) (end 174.112 116.537) (width 0.2) (layer "F.Cu") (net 17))
 (segment (start 173.625 90.325) (end 169.55 90.325) (width 0.2) (layer "F.Cu") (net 17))
 (segment (start 175.147 91.847) (end 173.625 90.325) (width 0.2) (layer "F.Cu") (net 17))
 (segment (start 174.112 116.537) (end 174.125 116.55) (width 0.2) (layer "F.Cu") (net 17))
 (segment (start 136.95 66.175) (end 169.55 66.175) (width 0.2) (layer "F.Cu") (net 24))
 (segment (start 135.29 71.84) (end 135.29 67.835) (width 0.2) (layer "F.Cu") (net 24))
 (segment (start 135.29 67.835) (end 136.95 66.175) (width 0.2) (layer "F.Cu") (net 24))
 (segment (start 138.575 67.175) (end 169.55 67.175) (width 0.2) (layer "F.Cu") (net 23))
 (segment (start 137.83 71.84) (end 137.83 67.92) (width 0.2) (layer "F.Cu") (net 23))
 (segment (start 137.83 67.92) (end 138.575 67.175) (width 0.2) (layer "F.Cu") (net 23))
 (segment (start 141.3 68.175) (end 169.55 68.175) (width 0.2) (layer "F.Cu") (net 22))
 (segment (start 140.37 71.84) (end 140.37 69.105) (width 0.2) (layer "F.Cu") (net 22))
 (segment (start 140.37 69.105) (end 141.3 68.175) (width 0.2) (layer "F.Cu") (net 22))
 (segment (start 126.210643 77.260643) (end 131.215 72.256285) (width 0.2) (layer "F.Cu") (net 3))
 (segment (start 116.3 93.8) (end 116.3 91.948715) (width 0.2) (layer "F.Cu") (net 3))
 (segment (start 124.981286 78.49) (end 126.210643 77.260643) (width 0.2) (layer "F.Cu") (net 3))
 (segment (start 131.215 66.66) (end 134.7 63.175) (width 0.2) (layer "F.Cu") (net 3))
 (segment (start 115.325 94.775) (end 116.3 93.8) (width 0.2) (layer "F.Cu") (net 3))
 (segment (start 120.915 78.49) (end 122.275 78.49) (width 0.2) (layer "F.Cu") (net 3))
 (segment (start 172.675 80.225) (end 172.675 82.025) (width 0.2) (layer "F.Cu") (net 3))
 (segment (start 109.89 92.16) (end 109.89 93.865) (width 0.2) (layer "F.Cu") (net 3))
 (segment (start 109.89 93.865) (end 110.8 94.775) (width 0.2) (layer "F.Cu") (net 3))
 (segment (start 172.675 82.025) (end 171.375 83.325) (width 0.2) (layer "F.Cu") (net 3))
 (segment (start 118.825 78.1253) (end 120.5503 78.1253) (width 0.2) (layer "F.Cu") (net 3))
 (segment (start 171.375 83.325) (end 169.55 83.325) (width 0.2) (layer "F.Cu") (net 3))
 (segment (start 110.8 94.775) (end 115.325 94.775) (width 0.2) (layer "F.Cu") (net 3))
 (segment (start 171.9 79.45) (end 172.675 80.225) (width 0.2) (layer "F.Cu") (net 3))
 (segment (start 112.3997 78.1253) (end 118.825 78.1253) (width 0.2) (layer "F.Cu") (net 3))
 (segment (start 134.7 63.175) (end 169.55 63.175) (width 0.2) (layer "F.Cu") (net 3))
 (segment (start 120.5503 78.1253) (end 120.915 78.49) (width 0.2) (layer "F.Cu") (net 3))
 (segment (start 128.798715 79.45) (end 171.9 79.45) (width 0.2) (layer "F.Cu") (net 3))
 (segment (start 131.215 72.256285) (end 131.215 66.66) (width 0.2) (layer "F.Cu") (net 3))
 (segment (start 109.89 80.635) (end 112.3997 78.1253) (width 0.2) (layer "F.Cu") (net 3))
 (segment (start 125.871285 77.6) (end 126.210643 77.260643) (width 0.2) (layer "F.Cu") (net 3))
 (segment (start 169.85 63.175) (end 169.55 63.175) (width 0.2) (layer "F.Cu") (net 3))
 (segment (start 116.3 91.948715) (end 128.798715 79.45) (width 0.2) (layer "F.Cu") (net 3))
 (segment (start 109.89 92.16) (end 109.89 80.635) (width 0.2) (layer "F.Cu") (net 3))
 (segment (start 122.275 78.49) (end 124.981286 78.49) (width 0.2) (layer "F.Cu") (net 3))
 (segment (start 130.21 67.71) (end 130.2 67.7) (width 0.2) (layer "F.Cu") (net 26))
 (segment (start 130.21 67.875) (end 130.21 67.71) (width 0.2) (layer "F.Cu") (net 26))
 (segment (start 134.425 62.175) (end 169.55 62.175) (width 0.2) (layer "F.Cu") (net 26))
 (segment (start 130.21 66.39) (end 134.425 62.175) (width 0.2) (layer "F.Cu") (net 26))
 (segment (start 130.21 71.84) (end 130.21 67.875) (width 0.2) (layer "F.Cu") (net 26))
 (segment (start 130.21 67.875) (end 130.21 66.39) (width 0.2) (layer "F.Cu") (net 26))
 (segment (start 127.67 67.755) (end 134.25 61.175) (width 0.2) (layer "F.Cu") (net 27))
 (segment (start 127.67 71.84) (end 127.67 67.755) (width 0.2) (layer "F.Cu") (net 27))
 (segment (start 134.25 61.175) (end 169.55 61.175) (width 0.2) (layer "F.Cu") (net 27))
 (segment (start 132.775 60.175) (end 169.55 60.175) (width 0.2) (layer "F.Cu") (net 28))
 (segment (start 125.13 71.84) (end 125.13 67.82) (width 0.2) (layer "F.Cu") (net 28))
 (segment (start 125.13 67.82) (end 132.775 60.175) (width 0.2) (layer "F.Cu") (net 28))
 (segment (start 132.75 67.925) (end 135.5 65.175) (width 0.2) (layer "F.Cu") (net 25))
 (segment (start 132.75 71.84) (end 132.75 67.925) (width 0.2) (layer "F.Cu") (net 25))
 (segment (start 135.5 65.175) (end 169.55 65.175) (width 0.2) (layer "F.Cu") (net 25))
 (segment (start 171.86601 121.617) (end 174.658 121.617) (width 0.2) (layer "F.Cu") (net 15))
 (segment (start 174.625 70.175) (end 169.55 70.175) (width 0.2) (layer "F.Cu") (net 15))
 (segment (start 176.55 72.1) (end 174.625 70.175) (width 0.2) (layer "F.Cu") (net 15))
 (segment (start 176.55 119.725) (end 176.55 72.1) (width 0.2) (layer "F.Cu") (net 15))
 (segment (start 174.658 121.617) (end 176.55 119.725) (width 0.2) (layer "F.Cu") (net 15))
 (segment (start 127.67 92.16) (end 137.505 82.325) (width 0.2) (layer "F.Cu") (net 36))
 (segment (start 137.505 82.325) (end 169.55 82.325) (width 0.2) (layer "F.Cu") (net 36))
 (segment (start 125.13 92.16) (end 135.965 81.325) (width 0.2) (layer "F.Cu") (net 37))
 (segment (start 135.965 81.325) (end 169.55 81.325) (width 0.2) (layer "F.Cu") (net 37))
 (segment (start 137.83 92.16) (end 141.665 88.325) (width 0.2) (layer "F.Cu") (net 32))
 (segment (start 141.665 88.325) (end 169.55 88.325) (width 0.2) (layer "F.Cu") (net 32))
 (segment (start 134.425 80.325) (end 169.55 80.325) (width 0.2) (layer "F.Cu") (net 38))
 (segment (start 122.59 92.16) (end 134.425 80.325) (width 0.2) (layer "F.Cu") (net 38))
 (segment (start 135.29 92.16) (end 140.125 87.325) (width 0.2) (layer "F.Cu") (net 33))
 (segment (start 140.125 87.325) (end 169.55 87.325) (width 0.2) (layer "F.Cu") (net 33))
 (segment (start 137.045 85.325) (end 169.55 85.325) (width 0.2) (layer "F.Cu") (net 35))
 (segment (start 130.21 92.16) (end 137.045 85.325) (width 0.2) (layer "F.Cu") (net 35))
 (segment (start 132.75 92.16) (end 138.585 86.325) (width 0.2) (layer "F.Cu") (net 34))
 (segment (start 138.585 86.325) (end 169.55 86.325) (width 0.2) (layer "F.Cu") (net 34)))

